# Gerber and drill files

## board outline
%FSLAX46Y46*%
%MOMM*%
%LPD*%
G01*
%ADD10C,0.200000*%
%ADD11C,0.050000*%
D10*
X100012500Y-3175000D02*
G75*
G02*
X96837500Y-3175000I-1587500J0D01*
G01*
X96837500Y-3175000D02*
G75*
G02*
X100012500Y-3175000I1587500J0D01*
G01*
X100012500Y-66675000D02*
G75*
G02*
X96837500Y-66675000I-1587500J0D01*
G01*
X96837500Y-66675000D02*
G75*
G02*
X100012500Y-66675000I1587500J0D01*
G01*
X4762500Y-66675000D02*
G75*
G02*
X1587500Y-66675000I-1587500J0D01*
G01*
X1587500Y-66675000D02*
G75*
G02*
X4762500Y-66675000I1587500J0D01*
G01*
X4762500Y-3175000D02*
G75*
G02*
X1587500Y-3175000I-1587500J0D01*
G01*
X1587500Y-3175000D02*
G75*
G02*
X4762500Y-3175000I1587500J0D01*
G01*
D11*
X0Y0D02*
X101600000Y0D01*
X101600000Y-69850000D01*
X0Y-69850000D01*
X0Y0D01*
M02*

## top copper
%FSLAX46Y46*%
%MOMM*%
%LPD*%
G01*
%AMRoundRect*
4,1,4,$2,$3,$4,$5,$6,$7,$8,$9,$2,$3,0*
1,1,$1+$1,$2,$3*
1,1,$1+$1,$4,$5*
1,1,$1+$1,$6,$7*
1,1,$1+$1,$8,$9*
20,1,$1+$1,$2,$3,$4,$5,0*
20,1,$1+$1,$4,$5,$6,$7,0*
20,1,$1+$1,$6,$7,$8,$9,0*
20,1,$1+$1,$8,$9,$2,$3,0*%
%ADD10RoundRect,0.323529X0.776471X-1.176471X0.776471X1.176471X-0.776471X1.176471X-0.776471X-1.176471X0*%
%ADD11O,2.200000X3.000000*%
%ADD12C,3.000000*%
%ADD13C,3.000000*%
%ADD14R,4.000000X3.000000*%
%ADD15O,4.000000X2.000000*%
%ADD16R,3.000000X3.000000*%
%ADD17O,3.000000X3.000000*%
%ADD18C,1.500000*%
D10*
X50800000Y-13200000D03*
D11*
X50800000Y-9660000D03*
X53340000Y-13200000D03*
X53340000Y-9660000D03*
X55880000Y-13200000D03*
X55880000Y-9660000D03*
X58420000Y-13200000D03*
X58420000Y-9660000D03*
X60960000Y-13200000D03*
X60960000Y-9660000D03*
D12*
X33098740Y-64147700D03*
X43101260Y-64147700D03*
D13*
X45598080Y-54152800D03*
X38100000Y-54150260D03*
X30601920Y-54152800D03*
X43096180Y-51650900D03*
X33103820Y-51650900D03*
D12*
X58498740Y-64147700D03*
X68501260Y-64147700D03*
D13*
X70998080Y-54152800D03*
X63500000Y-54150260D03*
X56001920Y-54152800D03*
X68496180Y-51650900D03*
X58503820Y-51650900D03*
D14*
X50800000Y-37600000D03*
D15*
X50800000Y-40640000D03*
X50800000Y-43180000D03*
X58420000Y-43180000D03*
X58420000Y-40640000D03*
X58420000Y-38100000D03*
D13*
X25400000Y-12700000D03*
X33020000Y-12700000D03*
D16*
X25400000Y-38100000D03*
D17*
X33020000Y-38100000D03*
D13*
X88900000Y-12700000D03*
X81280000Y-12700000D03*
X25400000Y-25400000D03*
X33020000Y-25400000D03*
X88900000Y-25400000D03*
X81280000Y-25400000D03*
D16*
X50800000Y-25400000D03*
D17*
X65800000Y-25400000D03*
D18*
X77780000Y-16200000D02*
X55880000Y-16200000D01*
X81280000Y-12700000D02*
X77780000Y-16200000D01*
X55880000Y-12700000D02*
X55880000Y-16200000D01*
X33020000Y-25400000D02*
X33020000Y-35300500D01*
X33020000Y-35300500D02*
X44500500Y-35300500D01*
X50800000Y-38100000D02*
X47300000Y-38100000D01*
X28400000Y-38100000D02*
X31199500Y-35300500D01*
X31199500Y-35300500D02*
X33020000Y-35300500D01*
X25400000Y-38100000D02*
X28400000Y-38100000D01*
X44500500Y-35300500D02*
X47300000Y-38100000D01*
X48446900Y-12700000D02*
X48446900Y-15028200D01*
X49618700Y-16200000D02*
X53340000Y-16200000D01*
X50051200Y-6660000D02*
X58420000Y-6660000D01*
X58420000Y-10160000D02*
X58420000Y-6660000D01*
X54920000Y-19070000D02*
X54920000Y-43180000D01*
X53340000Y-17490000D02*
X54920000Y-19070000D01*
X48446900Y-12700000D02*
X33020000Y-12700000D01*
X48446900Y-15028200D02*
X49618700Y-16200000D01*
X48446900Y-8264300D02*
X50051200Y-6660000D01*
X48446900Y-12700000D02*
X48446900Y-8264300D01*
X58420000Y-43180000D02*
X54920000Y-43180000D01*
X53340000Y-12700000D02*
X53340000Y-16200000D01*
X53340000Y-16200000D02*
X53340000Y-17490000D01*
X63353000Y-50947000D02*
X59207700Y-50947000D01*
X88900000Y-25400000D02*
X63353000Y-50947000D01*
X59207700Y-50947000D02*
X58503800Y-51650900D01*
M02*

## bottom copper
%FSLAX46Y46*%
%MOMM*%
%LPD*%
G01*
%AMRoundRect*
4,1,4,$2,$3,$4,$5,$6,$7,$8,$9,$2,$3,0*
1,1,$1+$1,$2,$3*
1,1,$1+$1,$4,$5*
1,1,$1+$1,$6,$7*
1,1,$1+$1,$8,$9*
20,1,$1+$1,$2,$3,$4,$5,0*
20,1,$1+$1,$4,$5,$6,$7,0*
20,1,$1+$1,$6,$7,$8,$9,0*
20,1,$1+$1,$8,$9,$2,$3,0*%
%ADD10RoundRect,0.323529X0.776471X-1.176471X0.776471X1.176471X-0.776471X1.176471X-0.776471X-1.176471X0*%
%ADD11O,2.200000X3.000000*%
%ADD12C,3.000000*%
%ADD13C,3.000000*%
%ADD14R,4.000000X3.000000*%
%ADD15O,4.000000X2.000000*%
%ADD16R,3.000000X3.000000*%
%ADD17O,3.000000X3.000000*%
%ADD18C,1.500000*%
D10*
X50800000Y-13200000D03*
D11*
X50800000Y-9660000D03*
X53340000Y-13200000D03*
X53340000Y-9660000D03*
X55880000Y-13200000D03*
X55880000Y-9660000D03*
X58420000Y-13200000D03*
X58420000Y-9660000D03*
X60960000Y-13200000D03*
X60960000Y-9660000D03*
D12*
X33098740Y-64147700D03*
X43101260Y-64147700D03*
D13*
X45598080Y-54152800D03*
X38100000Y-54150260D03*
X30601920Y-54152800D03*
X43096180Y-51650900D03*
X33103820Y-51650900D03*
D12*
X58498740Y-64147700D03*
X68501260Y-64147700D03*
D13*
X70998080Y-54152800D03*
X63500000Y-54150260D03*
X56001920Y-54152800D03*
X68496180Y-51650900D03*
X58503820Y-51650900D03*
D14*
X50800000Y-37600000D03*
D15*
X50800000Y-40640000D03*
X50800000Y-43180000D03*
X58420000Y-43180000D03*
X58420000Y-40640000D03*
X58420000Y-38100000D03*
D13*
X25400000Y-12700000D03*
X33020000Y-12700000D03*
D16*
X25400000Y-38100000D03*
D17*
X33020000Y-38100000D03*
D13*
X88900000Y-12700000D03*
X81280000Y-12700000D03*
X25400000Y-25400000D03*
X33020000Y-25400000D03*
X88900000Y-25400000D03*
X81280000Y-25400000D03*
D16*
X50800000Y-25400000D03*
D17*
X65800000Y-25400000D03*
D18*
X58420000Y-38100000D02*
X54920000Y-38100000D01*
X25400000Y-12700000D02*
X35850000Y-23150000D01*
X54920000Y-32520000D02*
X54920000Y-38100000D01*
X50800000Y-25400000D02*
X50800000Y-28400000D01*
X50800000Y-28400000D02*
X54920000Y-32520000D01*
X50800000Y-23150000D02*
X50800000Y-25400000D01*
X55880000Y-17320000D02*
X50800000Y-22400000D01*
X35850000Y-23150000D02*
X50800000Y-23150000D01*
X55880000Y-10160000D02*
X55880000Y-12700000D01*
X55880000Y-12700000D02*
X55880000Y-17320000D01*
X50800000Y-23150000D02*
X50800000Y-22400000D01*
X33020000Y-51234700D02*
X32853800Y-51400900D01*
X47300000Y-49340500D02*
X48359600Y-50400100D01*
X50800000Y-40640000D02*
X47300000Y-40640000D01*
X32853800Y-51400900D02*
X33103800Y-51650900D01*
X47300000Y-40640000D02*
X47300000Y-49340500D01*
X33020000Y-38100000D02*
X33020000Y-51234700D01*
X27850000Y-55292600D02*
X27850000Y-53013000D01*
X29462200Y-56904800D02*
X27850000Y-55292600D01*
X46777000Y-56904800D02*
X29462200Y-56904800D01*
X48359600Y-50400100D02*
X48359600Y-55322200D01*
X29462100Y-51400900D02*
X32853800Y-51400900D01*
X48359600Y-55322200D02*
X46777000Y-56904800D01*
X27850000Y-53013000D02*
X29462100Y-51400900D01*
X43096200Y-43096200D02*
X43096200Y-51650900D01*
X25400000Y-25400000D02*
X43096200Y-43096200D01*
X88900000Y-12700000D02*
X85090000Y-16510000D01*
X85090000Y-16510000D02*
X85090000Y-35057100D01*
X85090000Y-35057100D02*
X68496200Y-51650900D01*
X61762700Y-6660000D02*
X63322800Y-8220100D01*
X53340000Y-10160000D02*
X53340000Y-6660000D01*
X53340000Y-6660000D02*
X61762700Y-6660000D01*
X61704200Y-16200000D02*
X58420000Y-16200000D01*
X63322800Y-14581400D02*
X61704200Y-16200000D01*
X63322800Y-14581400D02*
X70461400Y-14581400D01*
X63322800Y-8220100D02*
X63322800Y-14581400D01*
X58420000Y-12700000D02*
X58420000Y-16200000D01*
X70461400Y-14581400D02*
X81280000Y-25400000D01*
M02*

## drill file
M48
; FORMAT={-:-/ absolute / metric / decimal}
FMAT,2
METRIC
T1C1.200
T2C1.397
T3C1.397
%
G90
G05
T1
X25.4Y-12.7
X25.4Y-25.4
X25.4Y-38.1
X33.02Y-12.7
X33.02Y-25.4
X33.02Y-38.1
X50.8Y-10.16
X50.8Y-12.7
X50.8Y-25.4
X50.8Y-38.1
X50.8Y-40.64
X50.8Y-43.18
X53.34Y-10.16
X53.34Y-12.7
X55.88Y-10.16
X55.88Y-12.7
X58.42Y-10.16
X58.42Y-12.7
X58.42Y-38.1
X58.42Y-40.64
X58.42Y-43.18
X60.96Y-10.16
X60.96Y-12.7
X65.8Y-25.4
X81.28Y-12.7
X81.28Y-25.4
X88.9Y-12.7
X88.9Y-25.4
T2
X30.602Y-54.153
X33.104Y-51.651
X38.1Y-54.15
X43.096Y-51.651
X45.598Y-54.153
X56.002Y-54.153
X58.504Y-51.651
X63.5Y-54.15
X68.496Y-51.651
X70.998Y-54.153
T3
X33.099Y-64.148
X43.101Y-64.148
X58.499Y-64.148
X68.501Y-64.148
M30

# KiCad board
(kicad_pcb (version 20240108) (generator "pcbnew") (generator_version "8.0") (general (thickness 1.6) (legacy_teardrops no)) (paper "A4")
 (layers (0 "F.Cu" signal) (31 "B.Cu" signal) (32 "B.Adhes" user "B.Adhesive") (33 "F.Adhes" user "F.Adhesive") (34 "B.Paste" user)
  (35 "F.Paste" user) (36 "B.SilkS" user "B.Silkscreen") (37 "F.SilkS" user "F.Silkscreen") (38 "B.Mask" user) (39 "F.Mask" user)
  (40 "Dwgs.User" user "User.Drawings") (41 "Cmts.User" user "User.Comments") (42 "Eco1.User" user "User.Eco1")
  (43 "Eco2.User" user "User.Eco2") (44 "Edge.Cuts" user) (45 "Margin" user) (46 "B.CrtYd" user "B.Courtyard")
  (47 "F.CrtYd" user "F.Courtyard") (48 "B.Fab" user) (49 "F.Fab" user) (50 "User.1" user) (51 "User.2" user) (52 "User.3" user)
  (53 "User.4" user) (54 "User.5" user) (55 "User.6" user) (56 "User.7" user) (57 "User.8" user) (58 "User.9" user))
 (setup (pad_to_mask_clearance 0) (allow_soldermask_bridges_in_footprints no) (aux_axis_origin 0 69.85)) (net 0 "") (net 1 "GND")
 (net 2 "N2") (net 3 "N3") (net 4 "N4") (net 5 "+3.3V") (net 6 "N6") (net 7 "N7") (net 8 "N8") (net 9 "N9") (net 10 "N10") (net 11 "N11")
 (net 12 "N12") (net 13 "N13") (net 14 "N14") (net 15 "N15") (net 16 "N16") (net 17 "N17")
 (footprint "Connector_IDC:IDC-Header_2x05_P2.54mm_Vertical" (layer "F.Cu") (at 50.8 12.7 90)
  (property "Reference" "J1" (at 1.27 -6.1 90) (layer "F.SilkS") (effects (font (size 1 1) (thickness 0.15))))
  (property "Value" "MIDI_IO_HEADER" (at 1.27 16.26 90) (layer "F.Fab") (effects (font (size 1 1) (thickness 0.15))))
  (pad "1" thru_hole roundrect (at 0 0 90) (size 3 2.2) (drill 1.2 (offset -0.5 0)) (layers "*.Cu" "*.Mask") (remove_unused_layers no)
   (roundrect_rratio 0.1470586364) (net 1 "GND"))
  (pad "2" thru_hole oval (at 2.54 0 90) (size 3 2.2) (drill 1.2 (offset 0.5 0)) (layers "*.Cu" "*.Mask") (remove_unused_layers no)
   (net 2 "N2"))
  (pad "3" thru_hole oval (at 0 2.54 90) (size 3 2.2) (drill 1.2 (offset -0.5 0)) (layers "*.Cu" "*.Mask") (remove_unused_layers no)
   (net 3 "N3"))
  (pad "4" thru_hole oval (at 2.54 2.54 90) (size 3 2.2) (drill 1.2 (offset 0.5 0)) (layers "*.Cu" "*.Mask") (remove_unused_layers no)
   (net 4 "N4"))
  (pad "5" thru_hole oval (at 0 5.08 90) (size 3 2.2) (drill 1.2 (offset -0.5 0)) (layers "*.Cu" "*.Mask") (remove_unused_layers no)
   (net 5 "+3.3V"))
  (pad "6" thru_hole oval (at 2.54 5.08 90) (size 3 2.2) (drill 1.2 (offset 0.5 0)) (layers "*.Cu" "*.Mask") (remove_unused_layers no)
   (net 5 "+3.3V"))
  (pad "7" thru_hole oval (at 0 7.62 90) (size 3 2.2) (drill 1.2 (offset -0.5 0)) (layers "*.Cu" "*.Mask") (remove_unused_layers no)
   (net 4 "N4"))
  (pad "8" thru_hole oval (at 2.54 7.62 90) (size 3 2.2) (drill 1.2 (offset 0.5 0)) (layers "*.Cu" "*.Mask") (remove_unused_layers no)
   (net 3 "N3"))
  (pad "9" thru_hole oval (at 0 10.16 90) (size 3 2.2) (drill 1.2 (offset -0.5 0)) (layers "*.Cu" "*.Mask") (remove_unused_layers no)
   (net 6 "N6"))
  (pad "10" thru_hole oval (at 2.54 10.16 90) (size 3 2.2) (drill 1.2 (offset 0.5 0)) (layers "*.Cu" "*.Mask") (remove_unused_layers no)
   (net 1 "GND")))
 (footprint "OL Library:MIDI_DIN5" (layer "F.Cu") (at 38.1 57.15)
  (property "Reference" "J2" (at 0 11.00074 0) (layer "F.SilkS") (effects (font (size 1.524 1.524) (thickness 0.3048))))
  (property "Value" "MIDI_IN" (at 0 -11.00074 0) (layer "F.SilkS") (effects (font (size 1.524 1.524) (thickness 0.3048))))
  (pad "" np_thru_hole circle (at -5.00126 6.9977) (size 3 3) (drill 1.397) (layers "F&B.Cu" "*.Mask" "F.SilkS"))
  (pad "" np_thru_hole circle (at 5.00126 6.9977) (size 3 3) (drill 1.397) (layers "F&B.Cu" "*.Mask" "F.SilkS"))
  (pad "1" thru_hole circle (at 7.49808 -2.9972) (size 3 3) (drill 1.397) (layers "*.Cu" "*.SilkS" "*.Mask") (remove_unused_layers no)
   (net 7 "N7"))
  (pad "2" thru_hole circle (at 0 -2.99974) (size 3 3) (drill 1.397) (layers "*.Cu" "*.SilkS" "*.Mask") (remove_unused_layers no)
   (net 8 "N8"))
  (pad "3" thru_hole circle (at -7.49808 -2.9972) (size 3 3) (drill 1.397) (layers "*.Cu" "*.SilkS" "*.Mask") (remove_unused_layers no)
   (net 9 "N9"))
  (pad "4" thru_hole circle (at 4.99618 -5.4991) (size 3 3) (drill 1.397) (layers "*.Cu" "*.SilkS" "*.Mask") (remove_unused_layers no)
   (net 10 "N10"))
  (pad "5" thru_hole circle (at -4.99618 -5.4991) (size 3 3) (drill 1.397) (layers "*.Cu" "*.SilkS" "*.Mask") (remove_unused_layers no)
   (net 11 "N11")))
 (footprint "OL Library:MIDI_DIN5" (layer "F.Cu") (at 63.5 57.15)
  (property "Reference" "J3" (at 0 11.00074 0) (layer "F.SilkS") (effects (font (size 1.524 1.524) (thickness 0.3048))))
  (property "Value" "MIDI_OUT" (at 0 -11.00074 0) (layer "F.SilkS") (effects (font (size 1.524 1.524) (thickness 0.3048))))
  (pad "" np_thru_hole circle (at -5.00126 6.9977) (size 3 3) (drill 1.397) (layers "F&B.Cu" "*.Mask" "F.SilkS"))
  (pad "" np_thru_hole circle (at 5.00126 6.9977) (size 3 3) (drill 1.397) (layers "F&B.Cu" "*.Mask" "F.SilkS"))
  (pad "1" thru_hole circle (at 7.49808 -2.9972) (size 3 3) (drill 1.397) (layers "*.Cu" "*.SilkS" "*.Mask") (remove_unused_layers no)
   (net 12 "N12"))
  (pad "2" thru_hole circle (at 0 -2.99974) (size 3 3) (drill 1.397) (layers "*.Cu" "*.SilkS" "*.Mask") (remove_unused_layers no)
   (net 1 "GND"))
  (pad "3" thru_hole circle (at -7.49808 -2.9972) (size 3 3) (drill 1.397) (layers "*.Cu" "*.SilkS" "*.Mask") (remove_unused_layers no)
   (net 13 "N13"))
  (pad "4" thru_hole circle (at 4.99618 -5.4991) (size 3 3) (drill 1.397) (layers "*.Cu" "*.SilkS" "*.Mask") (remove_unused_layers no)
   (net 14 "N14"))
  (pad "5" thru_hole circle (at -4.99618 -5.4991) (size 3 3) (drill 1.397) (layers "*.Cu" "*.SilkS" "*.Mask") (remove_unused_layers no)
   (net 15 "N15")))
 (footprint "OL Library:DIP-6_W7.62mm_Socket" (layer "F.Cu") (at 50.8 38.1)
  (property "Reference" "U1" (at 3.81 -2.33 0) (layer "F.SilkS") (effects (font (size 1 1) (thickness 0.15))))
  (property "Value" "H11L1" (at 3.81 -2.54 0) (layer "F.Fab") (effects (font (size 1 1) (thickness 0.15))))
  (pad "1" thru_hole rect (at 0 0) (size 4 3) (drill 1.2 (offset 0 -0.5)) (layers "*.Cu" "*.Mask") (remove_unused_layers no) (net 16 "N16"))
  (pad "2" thru_hole oval (at 0 2.54) (size 4 2) (drill 1.2) (layers "*.Cu" "*.Mask") (remove_unused_layers no) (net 11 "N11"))
  (pad "3" thru_hole oval (at 0 5.08) (size 4 2) (drill 1.2) (layers "*.Cu" "*.Mask") (remove_unused_layers no) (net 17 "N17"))
  (pad "4" thru_hole oval (at 7.62 5.08) (size 4 2) (drill 1.2) (layers "*.Cu" "*.Mask") (remove_unused_layers no) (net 3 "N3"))
  (pad "5" thru_hole oval (at 7.62 2.54) (size 4 2) (drill 1.2) (layers "*.Cu" "*.Mask") (remove_unused_layers no) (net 1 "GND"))
  (pad "6" thru_hole oval (at 7.62 0) (size 4 2) (drill 1.2) (layers "*.Cu" "*.Mask") (remove_unused_layers no) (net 5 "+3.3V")))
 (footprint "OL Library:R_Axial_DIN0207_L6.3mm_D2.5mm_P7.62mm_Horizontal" (layer "F.Cu") (at 25.4 12.7)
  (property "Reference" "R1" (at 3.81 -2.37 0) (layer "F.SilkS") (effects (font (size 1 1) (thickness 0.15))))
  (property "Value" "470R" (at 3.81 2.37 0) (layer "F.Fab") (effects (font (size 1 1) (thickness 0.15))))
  (pad "1" thru_hole circle (at 0 0) (size 3 3) (drill 1.2) (layers "*.Cu" "*.Mask") (remove_unused_layers no) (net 5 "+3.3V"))
  (pad "2" thru_hole circle (at 7.62 0) (size 3 3) (drill 1.2) (layers "*.Cu" "*.Mask") (remove_unused_layers no) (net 3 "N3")))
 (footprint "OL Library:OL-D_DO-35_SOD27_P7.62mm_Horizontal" (layer "F.Cu") (at 25.4 38.1)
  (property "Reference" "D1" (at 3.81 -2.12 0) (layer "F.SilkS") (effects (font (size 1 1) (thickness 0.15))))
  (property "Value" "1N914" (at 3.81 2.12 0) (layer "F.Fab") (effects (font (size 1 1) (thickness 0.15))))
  (pad "1" thru_hole rect (at 0 0) (size 3 3) (drill 1.2) (layers "*.Cu" "*.Mask") (remove_unused_layers no) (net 16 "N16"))
  (pad "2" thru_hole oval (at 7.62 0) (size 3 3) (drill 1.2) (layers "*.Cu" "*.Mask") (remove_unused_layers no) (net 11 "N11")))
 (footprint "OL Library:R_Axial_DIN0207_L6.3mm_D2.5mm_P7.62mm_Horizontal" (layer "F.Cu") (at 88.9 12.7 180)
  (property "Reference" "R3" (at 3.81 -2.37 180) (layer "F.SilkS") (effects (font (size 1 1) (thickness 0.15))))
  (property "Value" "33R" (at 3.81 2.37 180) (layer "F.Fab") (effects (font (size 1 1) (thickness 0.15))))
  (pad "1" thru_hole circle (at 0 0 180) (size 3 3) (drill 1.2) (layers "*.Cu" "*.Mask") (remove_unused_layers no) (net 14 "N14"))
  (pad "2" thru_hole circle (at 7.62 0 180) (size 3 3) (drill 1.2) (layers "*.Cu" "*.Mask") (remove_unused_layers no) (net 5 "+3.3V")))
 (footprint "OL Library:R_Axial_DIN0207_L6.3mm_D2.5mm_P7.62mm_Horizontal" (layer "F.Cu") (at 25.4 25.4)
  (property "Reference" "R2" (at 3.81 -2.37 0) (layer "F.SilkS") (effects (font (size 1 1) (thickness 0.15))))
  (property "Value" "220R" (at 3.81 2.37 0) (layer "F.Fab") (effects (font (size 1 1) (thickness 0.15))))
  (pad "1" thru_hole circle (at 0 0) (size 3 3) (drill 1.2) (layers "*.Cu" "*.Mask") (remove_unused_layers no) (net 10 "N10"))
  (pad "2" thru_hole circle (at 7.62 0) (size 3 3) (drill 1.2) (layers "*.Cu" "*.Mask") (remove_unused_layers no) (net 16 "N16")))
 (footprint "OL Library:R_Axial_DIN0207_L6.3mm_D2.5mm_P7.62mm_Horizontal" (layer "F.Cu") (at 88.9 25.4 180)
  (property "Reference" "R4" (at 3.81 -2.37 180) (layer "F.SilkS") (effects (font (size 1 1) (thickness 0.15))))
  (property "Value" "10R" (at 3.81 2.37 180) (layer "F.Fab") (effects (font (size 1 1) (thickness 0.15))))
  (pad "1" thru_hole circle (at 0 0 180) (size 3 3) (drill 1.2) (layers "*.Cu" "*.Mask") (remove_unused_layers no) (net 15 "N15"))
  (pad "2" thru_hole circle (at 7.62 0 180) (size 3 3) (drill 1.2) (layers "*.Cu" "*.Mask") (remove_unused_layers no) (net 4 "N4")))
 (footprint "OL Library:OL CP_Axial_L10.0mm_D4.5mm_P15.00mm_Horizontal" (layer "F.Cu") (at 50.8 25.4)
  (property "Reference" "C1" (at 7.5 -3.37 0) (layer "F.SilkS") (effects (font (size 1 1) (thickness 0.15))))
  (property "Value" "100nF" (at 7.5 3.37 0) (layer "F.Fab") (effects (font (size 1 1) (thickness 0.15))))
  (pad "1" thru_hole rect (at 0 0) (size 3 3) (drill 1.2) (layers "*.Cu" "*.Mask") (remove_unused_layers no) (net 5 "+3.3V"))
  (pad "2" thru_hole oval (at 15 0) (size 3 3) (drill 1.2) (layers "*.Cu" "*.Mask") (remove_unused_layers no) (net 1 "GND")))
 (gr_circle (center 98.425 3.175) (end 100.0125 3.175) (stroke (width 0.2) (type default)) (fill none) (layer "Edge.Cuts"))
 (gr_circle (center 98.425 66.675) (end 100.0125 66.675) (stroke (width 0.2) (type default)) (fill none) (layer "Edge.Cuts"))
 (gr_circle (center 3.175 66.675) (end 4.7625 66.675) (stroke (width 0.2) (type default)) (fill none) (layer "Edge.Cuts"))
 (gr_circle (center 3.175 3.175) (end 4.7625 3.175) (stroke (width 0.2) (type default)) (fill none) (layer "Edge.Cuts"))
 (gr_rect (start 0 0) (end 101.6 69.85) (locked yes) (stroke (width 0.05) (type default)) (fill none) (layer "Edge.Cuts"))
 (segment (start 77.78 16.2) (end 55.88 16.2) (width 1.5) (layer "F.Cu") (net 5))
 (segment (start 81.28 12.7) (end 77.78 16.2) (width 1.5) (layer "F.Cu") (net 5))
 (segment (start 55.88 12.7) (end 55.88 16.2) (width 1.5) (layer "F.Cu") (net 5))
 (segment (start 58.42 38.1) (end 54.92 38.1) (width 1.5) (layer "B.Cu") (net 5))
 (segment (start 25.4 12.7) (end 35.85 23.15) (width 1.5) (layer "B.Cu") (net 5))
 (segment (start 54.92 32.52) (end 54.92 38.1) (width 1.5) (layer "B.Cu") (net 5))
 (segment (start 50.8 25.4) (end 50.8 28.4) (width 1.5) (layer "B.Cu") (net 5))
 (segment (start 50.8 28.4) (end 54.92 32.52) (width 1.5) (layer "B.Cu") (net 5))
 (segment (start 50.8 23.15) (end 50.8 25.4) (width 1.5) (layer "B.Cu") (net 5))
 (segment (start 55.88 17.32) (end 50.8 22.4) (width 1.5) (layer "B.Cu") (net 5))
 (segment (start 35.85 23.15) (end 50.8 23.15) (width 1.5) (layer "B.Cu") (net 5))
 (segment (start 55.88 10.16) (end 55.88 12.7) (width 1.5) (layer "B.Cu") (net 5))
 (segment (start 55.88 12.7) (end 55.88 17.32) (width 1.5) (layer "B.Cu") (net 5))
 (segment (start 50.8 23.15) (end 50.8 22.4) (width 1.5) (layer "B.Cu") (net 5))
 (segment (start 33.02 25.4) (end 33.02 35.3005) (width 1.5) (layer "F.Cu") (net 16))
 (segment (start 33.02 35.3005) (end 44.5005 35.3005) (width 1.5) (layer "F.Cu") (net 16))
 (segment (start 50.8 38.1) (end 47.3 38.1) (width 1.5) (layer "F.Cu") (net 16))
 (segment (start 28.4 38.1) (end 31.1995 35.3005) (width 1.5) (layer "F.Cu") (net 16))
 (segment (start 31.1995 35.3005) (end 33.02 35.3005) (width 1.5) (layer "F.Cu") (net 16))
 (segment (start 25.4 38.1) (end 28.4 38.1) (width 1.5) (layer "F.Cu") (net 16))
 (segment (start 44.5005 35.3005) (end 47.3 38.1) (width 1.5) (layer "F.Cu") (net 16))
 (segment (start 33.02 51.2347) (end 32.8538 51.4009) (width 1.5) (layer "B.Cu") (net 11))
 (segment (start 47.3 49.3405) (end 48.3596 50.4001) (width 1.5) (layer "B.Cu") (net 11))
 (segment (start 50.8 40.64) (end 47.3 40.64) (width 1.5) (layer "B.Cu") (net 11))
 (segment (start 32.8538 51.4009) (end 33.1038 51.6509) (width 1.5) (layer "B.Cu") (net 11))
 (segment (start 47.3 40.64) (end 47.3 49.3405) (width 1.5) (layer "B.Cu") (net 11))
 (segment (start 33.02 38.1) (end 33.02 51.2347) (width 1.5) (layer "B.Cu") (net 11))
 (segment (start 27.85 55.2926) (end 27.85 53.013) (width 1.5) (layer "B.Cu") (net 11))
 (segment (start 29.4622 56.9048) (end 27.85 55.2926) (width 1.5) (layer "B.Cu") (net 11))
 (segment (start 46.777 56.9048) (end 29.4622 56.9048) (width 1.5) (layer "B.Cu") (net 11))
 (segment (start 48.3596 50.4001) (end 48.3596 55.3222) (width 1.5) (layer "B.Cu") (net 11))
 (segment (start 29.4621 51.4009) (end 32.8538 51.4009) (width 1.5) (layer "B.Cu") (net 11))
 (segment (start 48.3596 55.3222) (end 46.777 56.9048) (width 1.5) (layer "B.Cu") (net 11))
 (segment (start 27.85 53.013) (end 29.4621 51.4009) (width 1.5) (layer "B.Cu") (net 11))
 (segment (start 48.4469 12.7) (end 48.4469 15.0282) (width 1.5) (layer "F.Cu") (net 3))
 (segment (start 49.6187 16.2) (end 53.34 16.2) (width 1.5) (layer "F.Cu") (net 3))
 (segment (start 50.0512 6.66) (end 58.42 6.66) (width 1.5) (layer "F.Cu") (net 3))
 (segment (start 58.42 10.16) (end 58.42 6.66) (width 1.5) (layer "F.Cu") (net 3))
 (segment (start 54.92 19.07) (end 54.92 43.18) (width 1.5) (layer "F.Cu") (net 3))
 (segment (start 53.34 17.49) (end 54.92 19.07) (width 1.5) (layer "F.Cu") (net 3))
 (segment (start 48.4469 12.7) (end 33.02 12.7) (width 1.5) (layer "F.Cu") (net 3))
 (segment (start 48.4469 15.0282) (end 49.6187 16.2) (width 1.5) (layer "F.Cu") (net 3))
 (segment (start 48.4469 8.2643) (end 50.0512 6.66) (width 1.5) (layer "F.Cu") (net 3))
 (segment (start 48.4469 12.7) (end 48.4469 8.2643) (width 1.5) (layer "F.Cu") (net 3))
 (segment (start 58.42 43.18) (end 54.92 43.18) (width 1.5) (layer "F.Cu") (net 3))
 (segment (start 53.34 12.7) (end 53.34 16.2) (width 1.5) (layer "F.Cu") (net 3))
 (segment (start 53.34 16.2) (end 53.34 17.49) (width 1.5) (layer "F.Cu") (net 3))
 (segment (start 43.0962 43.0962) (end 43.0962 51.6509) (width 1.5) (layer "B.Cu") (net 10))
 (segment (start 25.4 25.4) (end 43.0962 43.0962) (width 1.5) (layer "B.Cu") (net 10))
 (segment (start 88.9 12.7) (end 85.09 16.51) (width 1.5) (layer "B.Cu") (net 14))
 (segment (start 85.09 16.51) (end 85.09 35.0571) (width 1.5) (layer "B.Cu") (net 14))
 (segment (start 85.09 35.0571) (end 68.4962 51.6509) (width 1.5) (layer "B.Cu") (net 14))
 (segment (start 61.7627 6.66) (end 63.3228 8.2201) (width 1.5) (layer "B.Cu") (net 4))
 (segment (start 53.34 10.16) (end 53.34 6.66) (width 1.5) (layer "B.Cu") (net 4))
 (segment (start 53.34 6.66) (end 61.7627 6.66) (width 1.5) (layer "B.Cu") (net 4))
 (segment (start 61.7042 16.2) (end 58.42 16.2) (width 1.5) (layer "B.Cu") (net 4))
 (segment (start 63.3228 14.5814) (end 61.7042 16.2) (width 1.5) (layer "B.Cu") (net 4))
 (segment (start 63.3228 14.5814) (end 70.4614 14.5814) (width 1.5) (layer "B.Cu") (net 4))
 (segment (start 63.3228 8.2201) (end 63.3228 14.5814) (width 1.5) (layer "B.Cu") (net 4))
 (segment (start 58.42 12.7) (end 58.42 16.2) (width 1.5) (layer "B.Cu") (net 4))
 (segment (start 70.4614 14.5814) (end 81.28 25.4) (width 1.5) (layer "B.Cu") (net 4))
 (segment (start 63.353 50.947) (end 59.2077 50.947) (width 1.5) (layer "F.Cu") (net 15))
 (segment (start 88.9 25.4) (end 63.353 50.947) (width 1.5) (layer "F.Cu") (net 15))
 (segment (start 59.2077 50.947) (end 58.5038 51.6509) (width 1.5) (layer "F.Cu") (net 15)))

